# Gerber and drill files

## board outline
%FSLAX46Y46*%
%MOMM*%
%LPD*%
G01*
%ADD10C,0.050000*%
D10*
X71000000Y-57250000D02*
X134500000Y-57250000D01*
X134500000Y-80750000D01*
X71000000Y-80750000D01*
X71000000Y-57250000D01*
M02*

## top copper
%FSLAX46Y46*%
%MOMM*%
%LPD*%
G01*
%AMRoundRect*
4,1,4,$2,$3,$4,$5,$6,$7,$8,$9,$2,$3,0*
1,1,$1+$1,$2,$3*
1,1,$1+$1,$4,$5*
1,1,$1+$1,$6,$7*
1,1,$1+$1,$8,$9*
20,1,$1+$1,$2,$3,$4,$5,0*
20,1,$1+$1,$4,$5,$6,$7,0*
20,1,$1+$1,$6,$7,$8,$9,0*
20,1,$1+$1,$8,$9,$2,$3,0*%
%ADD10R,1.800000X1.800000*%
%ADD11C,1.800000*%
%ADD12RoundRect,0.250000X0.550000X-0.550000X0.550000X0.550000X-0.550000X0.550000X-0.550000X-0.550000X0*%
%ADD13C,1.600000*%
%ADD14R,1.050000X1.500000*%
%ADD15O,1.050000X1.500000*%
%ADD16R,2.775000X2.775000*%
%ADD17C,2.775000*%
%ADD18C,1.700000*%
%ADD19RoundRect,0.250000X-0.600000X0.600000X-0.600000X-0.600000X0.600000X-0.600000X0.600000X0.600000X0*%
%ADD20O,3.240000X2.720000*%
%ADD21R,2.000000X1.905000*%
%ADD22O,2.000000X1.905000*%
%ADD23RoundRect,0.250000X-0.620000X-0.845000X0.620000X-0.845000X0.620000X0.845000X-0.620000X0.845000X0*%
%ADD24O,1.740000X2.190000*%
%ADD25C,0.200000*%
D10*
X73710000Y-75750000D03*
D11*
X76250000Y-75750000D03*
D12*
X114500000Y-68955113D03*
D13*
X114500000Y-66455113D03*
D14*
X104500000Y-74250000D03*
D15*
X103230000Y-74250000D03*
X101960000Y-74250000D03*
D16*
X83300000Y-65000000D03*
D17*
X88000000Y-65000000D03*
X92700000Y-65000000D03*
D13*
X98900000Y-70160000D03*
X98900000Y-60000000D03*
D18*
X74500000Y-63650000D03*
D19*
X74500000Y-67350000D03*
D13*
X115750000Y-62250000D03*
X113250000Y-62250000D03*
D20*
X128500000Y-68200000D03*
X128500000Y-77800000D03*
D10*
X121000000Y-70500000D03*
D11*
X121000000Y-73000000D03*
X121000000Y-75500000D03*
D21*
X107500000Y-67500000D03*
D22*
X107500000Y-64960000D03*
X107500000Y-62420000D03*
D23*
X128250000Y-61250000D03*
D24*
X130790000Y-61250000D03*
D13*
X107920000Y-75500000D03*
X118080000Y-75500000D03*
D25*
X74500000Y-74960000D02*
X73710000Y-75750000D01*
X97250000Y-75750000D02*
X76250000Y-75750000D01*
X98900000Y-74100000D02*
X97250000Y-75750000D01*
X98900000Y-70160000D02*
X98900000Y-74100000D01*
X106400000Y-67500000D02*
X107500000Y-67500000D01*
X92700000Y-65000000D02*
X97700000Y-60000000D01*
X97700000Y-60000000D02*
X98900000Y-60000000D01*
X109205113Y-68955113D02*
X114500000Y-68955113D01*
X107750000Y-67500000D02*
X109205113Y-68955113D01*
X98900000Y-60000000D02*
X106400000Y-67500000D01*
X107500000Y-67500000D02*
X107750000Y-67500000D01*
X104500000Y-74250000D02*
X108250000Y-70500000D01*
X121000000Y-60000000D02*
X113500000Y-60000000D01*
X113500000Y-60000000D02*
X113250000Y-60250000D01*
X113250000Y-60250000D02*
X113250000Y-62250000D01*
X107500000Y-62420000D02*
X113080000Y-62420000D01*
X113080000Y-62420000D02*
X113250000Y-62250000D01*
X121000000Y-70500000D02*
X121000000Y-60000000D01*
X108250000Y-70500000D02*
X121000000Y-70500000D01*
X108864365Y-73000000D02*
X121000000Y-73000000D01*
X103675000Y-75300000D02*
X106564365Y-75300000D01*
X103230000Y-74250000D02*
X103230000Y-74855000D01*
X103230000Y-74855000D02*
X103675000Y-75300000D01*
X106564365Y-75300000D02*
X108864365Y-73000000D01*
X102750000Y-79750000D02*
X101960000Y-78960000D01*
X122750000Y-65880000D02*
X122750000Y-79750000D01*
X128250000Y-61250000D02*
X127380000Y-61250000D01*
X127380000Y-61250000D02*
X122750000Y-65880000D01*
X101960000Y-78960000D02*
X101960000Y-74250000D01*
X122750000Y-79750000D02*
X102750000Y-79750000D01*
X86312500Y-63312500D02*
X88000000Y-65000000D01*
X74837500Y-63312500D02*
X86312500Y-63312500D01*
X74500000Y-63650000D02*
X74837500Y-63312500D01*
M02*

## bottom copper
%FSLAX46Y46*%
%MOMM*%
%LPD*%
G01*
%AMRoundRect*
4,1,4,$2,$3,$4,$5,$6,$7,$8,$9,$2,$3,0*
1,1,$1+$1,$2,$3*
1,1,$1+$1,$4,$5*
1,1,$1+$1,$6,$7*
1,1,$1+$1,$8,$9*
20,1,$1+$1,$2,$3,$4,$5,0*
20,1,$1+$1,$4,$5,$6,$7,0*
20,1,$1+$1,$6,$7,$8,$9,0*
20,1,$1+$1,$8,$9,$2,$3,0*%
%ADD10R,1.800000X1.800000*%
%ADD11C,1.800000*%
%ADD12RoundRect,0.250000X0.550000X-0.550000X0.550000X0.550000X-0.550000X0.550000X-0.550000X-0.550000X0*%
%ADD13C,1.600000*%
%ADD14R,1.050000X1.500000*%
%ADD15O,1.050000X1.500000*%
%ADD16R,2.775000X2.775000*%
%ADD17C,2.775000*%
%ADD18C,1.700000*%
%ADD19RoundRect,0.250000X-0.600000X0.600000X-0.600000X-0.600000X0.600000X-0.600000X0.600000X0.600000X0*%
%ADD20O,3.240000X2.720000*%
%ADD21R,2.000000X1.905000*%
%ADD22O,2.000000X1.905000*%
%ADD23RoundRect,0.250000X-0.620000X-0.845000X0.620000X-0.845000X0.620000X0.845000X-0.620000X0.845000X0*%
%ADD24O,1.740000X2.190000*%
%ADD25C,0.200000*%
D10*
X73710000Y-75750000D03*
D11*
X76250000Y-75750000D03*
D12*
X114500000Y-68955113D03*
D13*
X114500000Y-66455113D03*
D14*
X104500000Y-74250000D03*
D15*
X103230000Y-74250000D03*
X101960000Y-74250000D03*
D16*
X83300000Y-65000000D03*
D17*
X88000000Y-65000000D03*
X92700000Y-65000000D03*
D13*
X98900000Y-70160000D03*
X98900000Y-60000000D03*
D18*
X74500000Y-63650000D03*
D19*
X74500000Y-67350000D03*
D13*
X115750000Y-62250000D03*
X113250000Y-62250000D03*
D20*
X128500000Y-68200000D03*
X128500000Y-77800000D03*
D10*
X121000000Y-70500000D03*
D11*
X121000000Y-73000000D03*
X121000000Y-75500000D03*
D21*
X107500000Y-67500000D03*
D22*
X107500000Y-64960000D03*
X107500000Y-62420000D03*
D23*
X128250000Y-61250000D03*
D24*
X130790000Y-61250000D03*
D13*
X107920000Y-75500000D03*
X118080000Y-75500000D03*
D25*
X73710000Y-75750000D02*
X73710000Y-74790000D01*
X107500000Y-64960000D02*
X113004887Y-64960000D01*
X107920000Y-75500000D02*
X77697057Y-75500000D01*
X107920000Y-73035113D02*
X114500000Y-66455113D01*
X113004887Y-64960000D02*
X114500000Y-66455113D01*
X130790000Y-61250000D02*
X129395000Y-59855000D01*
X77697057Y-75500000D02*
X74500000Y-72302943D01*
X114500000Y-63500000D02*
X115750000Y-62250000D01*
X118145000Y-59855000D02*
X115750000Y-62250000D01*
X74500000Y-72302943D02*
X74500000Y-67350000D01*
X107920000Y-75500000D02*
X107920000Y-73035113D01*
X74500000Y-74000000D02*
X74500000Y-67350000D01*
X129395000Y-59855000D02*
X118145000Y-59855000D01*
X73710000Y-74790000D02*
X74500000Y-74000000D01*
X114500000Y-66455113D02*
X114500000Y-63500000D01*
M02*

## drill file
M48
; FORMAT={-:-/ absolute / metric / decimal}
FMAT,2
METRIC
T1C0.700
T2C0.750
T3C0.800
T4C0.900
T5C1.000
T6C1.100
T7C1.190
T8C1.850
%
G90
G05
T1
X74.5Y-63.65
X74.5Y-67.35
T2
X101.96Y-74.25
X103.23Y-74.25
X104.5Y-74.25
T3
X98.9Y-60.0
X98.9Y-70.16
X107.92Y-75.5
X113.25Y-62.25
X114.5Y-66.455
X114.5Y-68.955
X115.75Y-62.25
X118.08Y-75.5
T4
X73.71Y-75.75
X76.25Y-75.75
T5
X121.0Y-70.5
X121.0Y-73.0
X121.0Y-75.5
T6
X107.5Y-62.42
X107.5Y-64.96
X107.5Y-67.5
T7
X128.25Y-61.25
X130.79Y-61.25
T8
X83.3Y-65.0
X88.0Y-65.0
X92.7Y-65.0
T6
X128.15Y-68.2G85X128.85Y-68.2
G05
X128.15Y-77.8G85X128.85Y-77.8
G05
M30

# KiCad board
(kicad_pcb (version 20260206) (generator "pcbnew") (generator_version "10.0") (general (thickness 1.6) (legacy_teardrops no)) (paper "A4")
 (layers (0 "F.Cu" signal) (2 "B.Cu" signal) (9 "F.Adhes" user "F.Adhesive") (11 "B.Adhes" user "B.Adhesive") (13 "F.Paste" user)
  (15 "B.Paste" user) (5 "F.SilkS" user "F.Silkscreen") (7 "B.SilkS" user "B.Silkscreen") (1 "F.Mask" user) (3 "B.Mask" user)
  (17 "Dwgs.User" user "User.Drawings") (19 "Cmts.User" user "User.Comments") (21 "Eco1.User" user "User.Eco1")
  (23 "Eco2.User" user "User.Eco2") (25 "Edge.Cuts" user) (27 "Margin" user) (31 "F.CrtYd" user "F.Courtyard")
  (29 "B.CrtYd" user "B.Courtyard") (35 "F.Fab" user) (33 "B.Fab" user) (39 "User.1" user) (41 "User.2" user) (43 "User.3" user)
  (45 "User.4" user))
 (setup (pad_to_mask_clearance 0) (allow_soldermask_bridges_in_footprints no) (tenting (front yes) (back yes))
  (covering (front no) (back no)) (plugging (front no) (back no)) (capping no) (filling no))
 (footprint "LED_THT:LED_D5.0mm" (layer "F.Cu") (at 73.71 75.75)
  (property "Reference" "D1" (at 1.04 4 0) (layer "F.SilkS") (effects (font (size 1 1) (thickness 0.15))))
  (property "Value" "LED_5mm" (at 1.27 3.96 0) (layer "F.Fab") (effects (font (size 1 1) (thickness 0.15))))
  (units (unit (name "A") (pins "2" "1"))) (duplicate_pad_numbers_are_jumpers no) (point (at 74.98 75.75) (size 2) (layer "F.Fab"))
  (pad "1" thru_hole rect (at 0 0) (size 1.8 1.8) (drill 0.9) (layers "*.Cu" "*.Mask") (remove_unused_layers no) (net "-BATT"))
  (pad "2" thru_hole circle (at 2.54 0) (size 1.8 1.8) (drill 0.9) (layers "*.Cu" "*.Mask") (remove_unused_layers no) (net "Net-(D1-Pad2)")))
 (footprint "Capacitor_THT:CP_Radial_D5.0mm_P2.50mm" (layer "F.Cu") (at 114.5 68.955113 90)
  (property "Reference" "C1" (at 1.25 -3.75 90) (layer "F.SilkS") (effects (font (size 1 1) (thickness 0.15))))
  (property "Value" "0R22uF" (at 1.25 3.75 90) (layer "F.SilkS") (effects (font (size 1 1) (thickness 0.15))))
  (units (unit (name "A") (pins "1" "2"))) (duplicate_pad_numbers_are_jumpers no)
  (pad "1" thru_hole roundrect (at 0 0 90) (size 1.6 1.6) (drill 0.8) (layers "*.Cu" "*.Mask") (remove_unused_layers no)
   (roundrect_rratio 0.15625) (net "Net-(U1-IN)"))
  (pad "2" thru_hole circle (at 2.5 0 90) (size 1.6 1.6) (drill 0.8) (layers "*.Cu" "*.Mask") (remove_unused_layers no) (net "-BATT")))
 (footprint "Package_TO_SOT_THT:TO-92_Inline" (layer "F.Cu") (at 104.5 74.25 180)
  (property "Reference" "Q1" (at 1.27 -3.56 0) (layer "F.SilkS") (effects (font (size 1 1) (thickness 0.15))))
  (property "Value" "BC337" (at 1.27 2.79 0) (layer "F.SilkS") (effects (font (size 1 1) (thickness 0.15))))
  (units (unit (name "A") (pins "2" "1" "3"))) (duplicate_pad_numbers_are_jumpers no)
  (pad "1" thru_hole rect (at 0 0 180) (size 1.05 1.5) (drill 0.75) (layers "*.Cu" "*.Mask") (remove_unused_layers no) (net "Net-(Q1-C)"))
  (pad "2" thru_hole oval (at 1.27 0 180) (size 1.05 1.5) (drill 0.75) (layers "*.Cu" "*.Mask") (remove_unused_layers no) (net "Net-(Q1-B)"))
  (pad "3" thru_hole oval (at 2.54 0 180) (size 1.05 1.5) (drill 0.75) (layers "*.Cu" "*.Mask") (remove_unused_layers no)
   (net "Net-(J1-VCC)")))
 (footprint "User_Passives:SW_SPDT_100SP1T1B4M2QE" (layer "F.Cu") (at 88 65 90)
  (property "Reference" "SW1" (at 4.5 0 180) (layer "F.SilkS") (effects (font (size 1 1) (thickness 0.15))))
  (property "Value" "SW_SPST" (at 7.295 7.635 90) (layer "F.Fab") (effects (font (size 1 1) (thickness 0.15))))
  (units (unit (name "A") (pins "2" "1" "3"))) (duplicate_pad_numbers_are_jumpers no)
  (pad "1" thru_hole rect (at 0 -4.7 90) (size 2.775 2.775) (drill 1.85) (layers "*.Cu" "*.Mask") (remove_unused_layers no)
   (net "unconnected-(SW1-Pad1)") (solder_mask_margin 0.102))
  (pad "2" thru_hole circle (at 0 0 90) (size 2.775 2.775) (drill 1.85) (layers "*.Cu" "*.Mask") (remove_unused_layers no) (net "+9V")
   (solder_mask_margin 0.102))
  (pad "3" thru_hole circle (at 0 4.7 90) (size 2.775 2.775) (drill 1.85) (layers "*.Cu" "*.Mask") (remove_unused_layers no)
   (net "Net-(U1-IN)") (solder_mask_margin 0.102)))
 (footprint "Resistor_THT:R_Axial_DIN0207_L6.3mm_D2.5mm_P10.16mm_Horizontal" (layer "F.Cu") (at 98.9 70.16 90)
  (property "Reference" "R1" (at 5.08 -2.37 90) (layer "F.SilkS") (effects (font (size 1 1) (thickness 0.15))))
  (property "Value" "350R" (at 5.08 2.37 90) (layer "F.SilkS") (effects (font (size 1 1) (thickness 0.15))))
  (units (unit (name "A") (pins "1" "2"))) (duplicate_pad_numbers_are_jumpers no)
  (pad "1" thru_hole circle (at 0 0 90) (size 1.6 1.6) (drill 0.8) (layers "*.Cu" "*.Mask") (remove_unused_layers no) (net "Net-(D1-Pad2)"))
  (pad "2" thru_hole circle (at 10.16 0 90) (size 1.6 1.6) (drill 0.8) (layers "*.Cu" "*.Mask") (remove_unused_layers no)
   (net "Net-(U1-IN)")))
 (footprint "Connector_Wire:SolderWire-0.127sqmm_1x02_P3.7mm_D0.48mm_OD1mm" (layer "F.Cu") (at 74.5 63.65 -90)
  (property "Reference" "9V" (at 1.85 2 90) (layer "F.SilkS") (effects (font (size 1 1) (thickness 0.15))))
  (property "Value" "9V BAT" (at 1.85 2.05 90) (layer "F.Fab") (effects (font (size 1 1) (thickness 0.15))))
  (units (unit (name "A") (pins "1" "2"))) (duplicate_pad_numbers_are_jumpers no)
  (pad "1" thru_hole circle (at 0 0 270) (size 1.7 1.7) (drill 0.7) (layers "*.Cu" "*.Mask") (remove_unused_layers no) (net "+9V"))
  (pad "2" thru_hole roundrect (at 3.7 0 270) (size 1.7 1.7) (drill 0.7) (layers "*.Cu" "*.Mask") (remove_unused_layers no)
   (roundrect_rratio 0.1470588235) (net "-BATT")))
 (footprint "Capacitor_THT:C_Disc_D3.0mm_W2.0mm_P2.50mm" (layer "F.Cu") (at 115.75 62.25 180)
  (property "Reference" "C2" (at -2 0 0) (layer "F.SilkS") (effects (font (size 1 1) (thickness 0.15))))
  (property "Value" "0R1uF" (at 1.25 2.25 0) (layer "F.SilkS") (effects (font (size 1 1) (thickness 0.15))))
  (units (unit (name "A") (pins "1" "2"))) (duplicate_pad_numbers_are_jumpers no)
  (pad "1" thru_hole circle (at 0 0 180) (size 1.6 1.6) (drill 0.8) (layers "*.Cu" "*.Mask") (remove_unused_layers no) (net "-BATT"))
  (pad "2" thru_hole circle (at 2.5 0 180) (size 1.6 1.6) (drill 0.8) (layers "*.Cu" "*.Mask") (remove_unused_layers no) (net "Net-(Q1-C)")))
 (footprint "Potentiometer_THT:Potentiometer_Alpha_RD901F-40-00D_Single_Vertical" (layer "F.Cu") (at 121 70.5)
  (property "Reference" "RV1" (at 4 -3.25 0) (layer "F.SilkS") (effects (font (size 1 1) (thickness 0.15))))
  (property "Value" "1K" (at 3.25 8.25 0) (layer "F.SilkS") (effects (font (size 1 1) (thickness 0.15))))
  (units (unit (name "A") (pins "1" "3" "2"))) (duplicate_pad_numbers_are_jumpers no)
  (pad "" thru_hole oval (at 7.5 -2.3 90) (size 2.72 3.24) (drill oval 1.1 1.8) (layers "*.Cu" "*.Mask") (remove_unused_layers no))
  (pad "" thru_hole oval (at 7.5 7.3 90) (size 2.72 3.24) (drill oval 1.1 1.8) (layers "*.Cu" "*.Mask") (remove_unused_layers no))
  (pad "1" thru_hole rect (at 0 0 90) (size 1.8 1.8) (drill 1) (layers "*.Cu" "*.Mask") (remove_unused_layers no) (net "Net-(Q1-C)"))
  (pad "2" thru_hole circle (at 0 2.5 90) (size 1.8 1.8) (drill 1) (layers "*.Cu" "*.Mask") (remove_unused_layers no) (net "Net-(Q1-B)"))
  (pad "3" thru_hole circle (at 0 5 90) (size 1.8 1.8) (drill 1) (layers "*.Cu" "*.Mask") (remove_unused_layers no) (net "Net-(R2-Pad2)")))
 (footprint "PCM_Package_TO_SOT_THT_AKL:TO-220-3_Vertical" (layer "F.Cu") (at 107.5 67.5 90)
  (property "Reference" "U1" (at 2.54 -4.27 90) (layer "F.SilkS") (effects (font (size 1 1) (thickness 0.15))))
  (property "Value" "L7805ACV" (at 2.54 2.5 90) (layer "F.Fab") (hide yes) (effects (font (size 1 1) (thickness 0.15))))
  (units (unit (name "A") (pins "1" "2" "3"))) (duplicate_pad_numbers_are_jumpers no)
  (pad "1" thru_hole rect (at 0 0 90) (size 1.905 2) (drill 1.1) (layers "*.Cu" "*.Mask") (remove_unused_layers no) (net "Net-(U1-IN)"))
  (pad "2" thru_hole oval (at 2.54 0 90) (size 1.905 2) (drill 1.1) (layers "*.Cu" "*.Mask") (remove_unused_layers no) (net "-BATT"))
  (pad "3" thru_hole oval (at 5.08 0 90) (size 1.905 2) (drill 1.1) (layers "*.Cu" "*.Mask") (remove_unused_layers no) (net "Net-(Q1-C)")))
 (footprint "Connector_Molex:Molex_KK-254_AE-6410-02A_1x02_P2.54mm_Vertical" (layer "F.Cu") (at 128.25 61.25)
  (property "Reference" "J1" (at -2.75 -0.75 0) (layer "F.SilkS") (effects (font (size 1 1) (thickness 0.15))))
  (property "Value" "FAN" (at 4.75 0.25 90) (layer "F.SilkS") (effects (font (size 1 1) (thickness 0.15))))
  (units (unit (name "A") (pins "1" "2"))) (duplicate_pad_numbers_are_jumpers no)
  (pad "1" thru_hole roundrect (at 0 0) (size 1.74 2.19) (drill 1.19) (layers "*.Cu" "*.Mask") (remove_unused_layers no)
   (roundrect_rratio 0.143678) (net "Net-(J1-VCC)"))
  (pad "2" thru_hole oval (at 2.54 0) (size 1.74 2.19) (drill 1.19) (layers "*.Cu" "*.Mask") (remove_unused_layers no) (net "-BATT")))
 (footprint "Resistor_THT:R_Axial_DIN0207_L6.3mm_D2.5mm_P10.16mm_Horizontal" (layer "F.Cu") (at 107.92 75.5)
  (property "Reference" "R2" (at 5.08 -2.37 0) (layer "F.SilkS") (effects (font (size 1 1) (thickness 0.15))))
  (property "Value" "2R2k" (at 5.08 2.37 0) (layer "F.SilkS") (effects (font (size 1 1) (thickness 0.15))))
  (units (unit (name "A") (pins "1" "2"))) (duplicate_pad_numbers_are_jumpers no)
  (pad "1" thru_hole circle (at 0 0) (size 1.6 1.6) (drill 0.8) (layers "*.Cu" "*.Mask") (remove_unused_layers no) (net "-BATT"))
  (pad "2" thru_hole circle (at 10.16 0) (size 1.6 1.6) (drill 0.8) (layers "*.Cu" "*.Mask") (remove_unused_layers no) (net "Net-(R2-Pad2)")))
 (gr_rect (start 71 57.25) (end 134.5 80.75) (stroke (width 0.05) (type default)) (fill no) (layer "Edge.Cuts"))
 (segment (start 74.5 74.96) (end 73.71 75.75) (width 0.2) (layer "F.Cu") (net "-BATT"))
 (segment (start 73.71 75.75) (end 73.71 74.79) (width 0.2) (layer "B.Cu") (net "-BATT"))
 (segment (start 107.5 64.96) (end 113.004887 64.96) (width 0.2) (layer "B.Cu") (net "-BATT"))
 (segment (start 107.92 75.5) (end 77.697057 75.5) (width 0.2) (layer "B.Cu") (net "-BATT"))
 (segment (start 107.92 73.035113) (end 114.5 66.455113) (width 0.2) (layer "B.Cu") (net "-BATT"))
 (segment (start 113.004887 64.96) (end 114.5 66.455113) (width 0.2) (layer "B.Cu") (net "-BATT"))
 (segment (start 130.79 61.25) (end 129.395 59.855) (width 0.2) (layer "B.Cu") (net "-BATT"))
 (segment (start 77.697057 75.5) (end 74.5 72.302943) (width 0.2) (layer "B.Cu") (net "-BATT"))
 (segment (start 114.5 63.5) (end 115.75 62.25) (width 0.2) (layer "B.Cu") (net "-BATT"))
 (segment (start 118.145 59.855) (end 115.75 62.25) (width 0.2) (layer "B.Cu") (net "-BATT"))
 (segment (start 74.5 72.302943) (end 74.5 67.35) (width 0.2) (layer "B.Cu") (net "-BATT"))
 (segment (start 107.92 75.5) (end 107.92 73.035113) (width 0.2) (layer "B.Cu") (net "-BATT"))
 (segment (start 74.5 74) (end 74.5 67.35) (width 0.2) (layer "B.Cu") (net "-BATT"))
 (segment (start 129.395 59.855) (end 118.145 59.855) (width 0.2) (layer "B.Cu") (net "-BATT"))
 (segment (start 73.71 74.79) (end 74.5 74) (width 0.2) (layer "B.Cu") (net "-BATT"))
 (segment (start 114.5 66.455113) (end 114.5 63.5) (width 0.2) (layer "B.Cu") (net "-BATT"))
 (segment (start 97.25 75.75) (end 76.25 75.75) (width 0.2) (layer "F.Cu") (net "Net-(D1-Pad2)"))
 (segment (start 98.9 74.1) (end 97.25 75.75) (width 0.2) (layer "F.Cu") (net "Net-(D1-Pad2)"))
 (segment (start 98.9 70.16) (end 98.9 74.1) (width 0.2) (layer "F.Cu") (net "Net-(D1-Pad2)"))
 (segment (start 106.4 67.5) (end 107.5 67.5) (width 0.2) (layer "F.Cu") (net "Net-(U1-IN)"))
 (segment (start 92.7 65) (end 97.7 60) (width 0.2) (layer "F.Cu") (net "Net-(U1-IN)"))
 (segment (start 97.7 60) (end 98.9 60) (width 0.2) (layer "F.Cu") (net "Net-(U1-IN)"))
 (segment (start 109.205113 68.955113) (end 114.5 68.955113) (width 0.2) (layer "F.Cu") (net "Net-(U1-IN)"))
 (segment (start 107.75 67.5) (end 109.205113 68.955113) (width 0.2) (layer "F.Cu") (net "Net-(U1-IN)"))
 (segment (start 98.9 60) (end 106.4 67.5) (width 0.2) (layer "F.Cu") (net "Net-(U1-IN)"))
 (segment (start 107.5 67.5) (end 107.75 67.5) (width 0.2) (layer "F.Cu") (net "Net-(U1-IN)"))
 (segment (start 104.5 74.25) (end 108.25 70.5) (width 0.2) (layer "F.Cu") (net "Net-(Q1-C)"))
 (segment (start 121 60) (end 113.5 60) (width 0.2) (layer "F.Cu") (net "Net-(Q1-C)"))
 (segment (start 113.5 60) (end 113.25 60.25) (width 0.2) (layer "F.Cu") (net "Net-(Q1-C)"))
 (segment (start 113.25 60.25) (end 113.25 62.25) (width 0.2) (layer "F.Cu") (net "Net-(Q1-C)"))
 (segment (start 107.5 62.42) (end 113.08 62.42) (width 0.2) (layer "F.Cu") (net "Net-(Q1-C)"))
 (segment (start 113.08 62.42) (end 113.25 62.25) (width 0.2) (layer "F.Cu") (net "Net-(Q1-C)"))
 (segment (start 121 70.5) (end 121 60) (width 0.2) (layer "F.Cu") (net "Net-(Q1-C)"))
 (segment (start 108.25 70.5) (end 121 70.5) (width 0.2) (layer "F.Cu") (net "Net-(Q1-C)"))
 (segment (start 108.864365 73) (end 121 73) (width 0.2) (layer "F.Cu") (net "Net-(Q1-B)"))
 (segment (start 103.675 75.3) (end 106.564365 75.3) (width 0.2) (layer "F.Cu") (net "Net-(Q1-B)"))
 (segment (start 103.23 74.25) (end 103.23 74.855) (width 0.2) (layer "F.Cu") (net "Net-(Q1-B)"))
 (segment (start 103.23 74.855) (end 103.675 75.3) (width 0.2) (layer "F.Cu") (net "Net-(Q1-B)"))
 (segment (start 106.564365 75.3) (end 108.864365 73) (width 0.2) (layer "F.Cu") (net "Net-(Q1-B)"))
 (segment (start 102.75 79.75) (end 101.96 78.96) (width 0.2) (layer "F.Cu") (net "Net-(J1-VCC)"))
 (segment (start 122.75 65.88) (end 122.75 79.75) (width 0.2) (layer "F.Cu") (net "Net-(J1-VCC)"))
 (segment (start 128.25 61.25) (end 127.38 61.25) (width 0.2) (layer "F.Cu") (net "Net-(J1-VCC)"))
 (segment (start 127.38 61.25) (end 122.75 65.88) (width 0.2) (layer "F.Cu") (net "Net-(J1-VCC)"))
 (segment (start 101.96 78.96) (end 101.96 74.25) (width 0.2) (layer "F.Cu") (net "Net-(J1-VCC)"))
 (segment (start 122.75 79.75) (end 102.75 79.75) (width 0.2) (layer "F.Cu") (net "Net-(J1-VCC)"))
 (segment (start 86.3125 63.3125) (end 88 65) (width 0.2) (layer "F.Cu") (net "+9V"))
 (segment (start 74.8375 63.3125) (end 86.3125 63.3125) (width 0.2) (layer "F.Cu") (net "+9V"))
 (segment (start 74.5 63.65) (end 74.8375 63.3125) (width 0.2) (layer "F.Cu") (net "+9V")))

